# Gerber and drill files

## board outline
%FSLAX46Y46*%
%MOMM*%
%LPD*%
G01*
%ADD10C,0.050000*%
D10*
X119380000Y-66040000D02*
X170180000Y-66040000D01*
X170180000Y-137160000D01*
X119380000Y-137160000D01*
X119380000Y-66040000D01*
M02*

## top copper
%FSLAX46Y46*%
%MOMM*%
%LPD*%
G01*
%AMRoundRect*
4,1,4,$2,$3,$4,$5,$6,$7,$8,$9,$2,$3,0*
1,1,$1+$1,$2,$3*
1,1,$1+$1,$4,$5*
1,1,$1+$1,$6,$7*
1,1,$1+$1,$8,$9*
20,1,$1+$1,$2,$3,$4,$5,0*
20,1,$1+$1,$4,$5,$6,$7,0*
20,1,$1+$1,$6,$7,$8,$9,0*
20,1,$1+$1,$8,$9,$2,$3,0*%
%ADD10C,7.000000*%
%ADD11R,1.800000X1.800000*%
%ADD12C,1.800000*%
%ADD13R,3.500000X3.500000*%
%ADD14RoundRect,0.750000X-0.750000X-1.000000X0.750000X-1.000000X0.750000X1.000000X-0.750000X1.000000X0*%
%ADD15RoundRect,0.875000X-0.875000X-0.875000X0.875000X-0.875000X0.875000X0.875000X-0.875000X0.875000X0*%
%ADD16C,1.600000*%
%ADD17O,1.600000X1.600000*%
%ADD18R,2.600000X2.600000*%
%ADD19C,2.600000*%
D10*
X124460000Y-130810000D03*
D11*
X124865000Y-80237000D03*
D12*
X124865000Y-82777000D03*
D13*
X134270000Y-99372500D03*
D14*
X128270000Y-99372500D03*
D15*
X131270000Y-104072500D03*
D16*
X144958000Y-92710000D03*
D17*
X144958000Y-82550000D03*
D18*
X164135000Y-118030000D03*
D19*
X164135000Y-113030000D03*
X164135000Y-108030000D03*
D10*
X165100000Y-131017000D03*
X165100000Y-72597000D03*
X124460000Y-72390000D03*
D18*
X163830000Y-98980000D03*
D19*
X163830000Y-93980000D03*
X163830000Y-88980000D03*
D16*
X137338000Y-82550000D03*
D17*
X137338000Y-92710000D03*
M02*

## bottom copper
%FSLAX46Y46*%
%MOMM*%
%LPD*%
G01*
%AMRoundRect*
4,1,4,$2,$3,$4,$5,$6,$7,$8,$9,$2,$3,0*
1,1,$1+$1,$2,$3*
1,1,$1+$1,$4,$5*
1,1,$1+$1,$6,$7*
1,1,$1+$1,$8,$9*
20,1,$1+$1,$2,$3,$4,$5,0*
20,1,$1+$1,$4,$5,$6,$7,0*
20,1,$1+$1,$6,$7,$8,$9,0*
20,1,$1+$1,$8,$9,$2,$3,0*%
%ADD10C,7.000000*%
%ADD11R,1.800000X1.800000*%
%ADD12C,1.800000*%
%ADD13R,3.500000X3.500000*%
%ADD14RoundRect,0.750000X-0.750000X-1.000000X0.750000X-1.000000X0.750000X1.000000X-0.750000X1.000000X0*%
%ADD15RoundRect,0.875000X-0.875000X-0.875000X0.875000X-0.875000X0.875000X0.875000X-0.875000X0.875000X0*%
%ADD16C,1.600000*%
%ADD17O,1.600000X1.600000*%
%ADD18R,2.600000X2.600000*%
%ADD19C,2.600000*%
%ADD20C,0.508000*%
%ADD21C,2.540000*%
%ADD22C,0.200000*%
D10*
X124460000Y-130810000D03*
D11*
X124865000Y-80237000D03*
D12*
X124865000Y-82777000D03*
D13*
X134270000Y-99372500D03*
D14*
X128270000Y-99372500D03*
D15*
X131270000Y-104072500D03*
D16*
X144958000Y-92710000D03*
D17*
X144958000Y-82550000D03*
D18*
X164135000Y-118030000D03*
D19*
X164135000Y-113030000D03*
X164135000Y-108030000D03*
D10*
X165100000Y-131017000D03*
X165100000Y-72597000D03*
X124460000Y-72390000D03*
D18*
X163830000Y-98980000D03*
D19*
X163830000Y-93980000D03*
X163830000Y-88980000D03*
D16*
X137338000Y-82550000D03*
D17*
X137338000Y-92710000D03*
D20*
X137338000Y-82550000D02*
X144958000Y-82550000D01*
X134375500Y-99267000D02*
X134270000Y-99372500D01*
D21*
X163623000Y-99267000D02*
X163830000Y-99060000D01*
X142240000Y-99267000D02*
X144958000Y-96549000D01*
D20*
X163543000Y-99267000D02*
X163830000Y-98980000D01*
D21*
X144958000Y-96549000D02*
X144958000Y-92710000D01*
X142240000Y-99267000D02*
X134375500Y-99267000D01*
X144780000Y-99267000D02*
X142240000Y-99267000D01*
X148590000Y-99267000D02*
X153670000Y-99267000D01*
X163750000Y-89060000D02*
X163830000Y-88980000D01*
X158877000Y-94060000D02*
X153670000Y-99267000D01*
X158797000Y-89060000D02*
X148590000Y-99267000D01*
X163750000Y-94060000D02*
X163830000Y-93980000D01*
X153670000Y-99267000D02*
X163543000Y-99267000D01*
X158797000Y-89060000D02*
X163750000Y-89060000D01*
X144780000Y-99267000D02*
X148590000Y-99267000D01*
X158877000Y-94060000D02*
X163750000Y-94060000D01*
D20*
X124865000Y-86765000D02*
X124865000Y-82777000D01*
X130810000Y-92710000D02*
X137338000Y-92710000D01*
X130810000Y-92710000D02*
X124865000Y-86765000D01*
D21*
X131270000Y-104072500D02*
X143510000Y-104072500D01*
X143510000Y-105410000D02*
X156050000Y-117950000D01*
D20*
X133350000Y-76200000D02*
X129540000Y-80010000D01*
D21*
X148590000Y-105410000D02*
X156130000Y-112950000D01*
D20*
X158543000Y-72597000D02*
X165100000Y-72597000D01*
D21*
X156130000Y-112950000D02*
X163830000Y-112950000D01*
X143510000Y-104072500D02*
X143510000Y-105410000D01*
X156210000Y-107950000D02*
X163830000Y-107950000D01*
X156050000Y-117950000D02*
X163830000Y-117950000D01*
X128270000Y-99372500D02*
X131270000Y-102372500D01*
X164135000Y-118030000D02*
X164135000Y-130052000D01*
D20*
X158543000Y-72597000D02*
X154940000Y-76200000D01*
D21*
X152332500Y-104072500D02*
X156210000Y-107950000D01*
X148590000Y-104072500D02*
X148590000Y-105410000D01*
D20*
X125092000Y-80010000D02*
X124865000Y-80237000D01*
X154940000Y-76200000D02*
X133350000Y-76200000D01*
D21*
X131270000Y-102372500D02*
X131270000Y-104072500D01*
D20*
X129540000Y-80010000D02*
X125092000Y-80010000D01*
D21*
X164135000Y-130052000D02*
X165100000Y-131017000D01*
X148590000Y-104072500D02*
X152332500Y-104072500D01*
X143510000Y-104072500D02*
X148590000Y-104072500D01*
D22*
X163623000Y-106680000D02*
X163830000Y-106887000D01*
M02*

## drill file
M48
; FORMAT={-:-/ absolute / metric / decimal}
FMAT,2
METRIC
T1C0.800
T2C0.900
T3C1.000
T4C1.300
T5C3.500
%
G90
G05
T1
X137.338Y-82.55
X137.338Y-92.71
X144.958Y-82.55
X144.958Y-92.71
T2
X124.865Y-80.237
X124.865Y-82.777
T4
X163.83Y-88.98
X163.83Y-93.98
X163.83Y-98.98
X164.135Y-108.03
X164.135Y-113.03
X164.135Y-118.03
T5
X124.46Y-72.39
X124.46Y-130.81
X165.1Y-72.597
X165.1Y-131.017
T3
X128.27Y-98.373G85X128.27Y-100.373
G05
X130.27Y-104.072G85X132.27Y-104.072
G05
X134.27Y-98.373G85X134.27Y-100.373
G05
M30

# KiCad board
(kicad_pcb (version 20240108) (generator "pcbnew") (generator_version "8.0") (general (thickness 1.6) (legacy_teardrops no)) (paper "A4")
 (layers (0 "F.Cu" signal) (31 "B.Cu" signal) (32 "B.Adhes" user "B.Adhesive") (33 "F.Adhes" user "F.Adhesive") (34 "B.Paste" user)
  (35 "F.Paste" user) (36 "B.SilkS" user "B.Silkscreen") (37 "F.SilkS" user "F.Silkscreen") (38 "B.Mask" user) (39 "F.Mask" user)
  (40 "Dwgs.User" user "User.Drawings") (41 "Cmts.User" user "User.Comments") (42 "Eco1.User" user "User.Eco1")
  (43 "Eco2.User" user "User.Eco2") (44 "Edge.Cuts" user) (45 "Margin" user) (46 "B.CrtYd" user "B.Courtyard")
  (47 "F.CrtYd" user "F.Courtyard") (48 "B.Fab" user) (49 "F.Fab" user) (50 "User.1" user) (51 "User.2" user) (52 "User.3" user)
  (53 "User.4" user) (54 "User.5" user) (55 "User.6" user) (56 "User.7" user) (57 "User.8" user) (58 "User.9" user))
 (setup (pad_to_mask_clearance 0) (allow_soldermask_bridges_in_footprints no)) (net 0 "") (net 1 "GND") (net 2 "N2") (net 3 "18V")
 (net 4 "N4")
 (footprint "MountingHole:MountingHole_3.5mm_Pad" (layer "F.Cu") (at 124.46 130.81)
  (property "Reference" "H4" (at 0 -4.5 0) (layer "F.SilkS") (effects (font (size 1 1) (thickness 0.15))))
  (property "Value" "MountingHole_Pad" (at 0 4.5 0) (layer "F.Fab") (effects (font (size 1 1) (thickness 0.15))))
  (pad "1" thru_hole circle (at 0 0) (size 7 7) (drill 3.5) (layers "*.Cu" "*.Mask") (remove_unused_layers no) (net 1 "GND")))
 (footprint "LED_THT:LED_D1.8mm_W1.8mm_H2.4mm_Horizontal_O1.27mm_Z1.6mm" (layer "F.Cu") (at 124.865 80.237 -90)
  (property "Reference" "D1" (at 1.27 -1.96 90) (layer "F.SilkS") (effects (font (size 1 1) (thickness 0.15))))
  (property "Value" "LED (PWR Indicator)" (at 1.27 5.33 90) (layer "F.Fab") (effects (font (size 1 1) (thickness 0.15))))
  (pad "1" thru_hole rect (at 0 0 270) (size 1.8 1.8) (drill 0.9) (layers "*.Cu" "*.Mask") (remove_unused_layers no) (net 1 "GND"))
  (pad "2" thru_hole circle (at 2.54 0 270) (size 1.8 1.8) (drill 0.9) (layers "*.Cu" "*.Mask") (remove_unused_layers no) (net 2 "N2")))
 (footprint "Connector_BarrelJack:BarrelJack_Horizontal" (layer "F.Cu") (at 134.27 99.3725)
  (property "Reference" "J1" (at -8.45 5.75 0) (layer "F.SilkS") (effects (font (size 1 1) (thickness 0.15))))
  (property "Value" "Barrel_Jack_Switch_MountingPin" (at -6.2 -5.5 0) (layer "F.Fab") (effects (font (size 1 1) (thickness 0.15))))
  (pad "1" thru_hole rect (at 0 0) (size 3.5 3.5) (drill oval 1 3) (layers "*.Cu" "*.Mask") (remove_unused_layers no) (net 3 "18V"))
  (pad "2" thru_hole roundrect (at -6 0) (size 3 3.5) (drill oval 1 3) (layers "*.Cu" "*.Mask") (remove_unused_layers no)
   (roundrect_rratio 0.25) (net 1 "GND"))
  (pad "3" thru_hole roundrect (at -3 4.7) (size 3.5 3.5) (drill oval 3 1) (layers "*.Cu" "*.Mask") (remove_unused_layers no)
   (roundrect_rratio 0.25) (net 1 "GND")))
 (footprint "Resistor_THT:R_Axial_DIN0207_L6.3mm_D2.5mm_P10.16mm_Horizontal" (layer "F.Cu") (at 144.958 92.71 90)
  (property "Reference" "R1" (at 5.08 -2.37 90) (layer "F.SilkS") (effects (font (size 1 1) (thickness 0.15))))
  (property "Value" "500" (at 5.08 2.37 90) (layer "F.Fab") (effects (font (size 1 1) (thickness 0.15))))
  (pad "1" thru_hole circle (at 0 0 90) (size 1.6 1.6) (drill 0.8) (layers "*.Cu" "*.Mask") (remove_unused_layers no) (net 3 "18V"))
  (pad "2" thru_hole oval (at 10.16 0 90) (size 1.6 1.6) (drill 0.8) (layers "*.Cu" "*.Mask") (remove_unused_layers no) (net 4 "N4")))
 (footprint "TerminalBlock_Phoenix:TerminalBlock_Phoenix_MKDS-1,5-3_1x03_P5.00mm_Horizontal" (layer "F.Cu") (at 164.135 118.03 90)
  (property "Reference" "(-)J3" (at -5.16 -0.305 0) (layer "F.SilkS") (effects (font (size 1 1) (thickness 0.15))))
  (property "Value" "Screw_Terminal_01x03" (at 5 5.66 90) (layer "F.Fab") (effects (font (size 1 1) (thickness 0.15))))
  (pad "1" thru_hole rect (at 0 0 90) (size 2.6 2.6) (drill 1.3) (layers "*.Cu" "*.Mask") (remove_unused_layers no) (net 1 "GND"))
  (pad "2" thru_hole circle (at 5 0 90) (size 2.6 2.6) (drill 1.3) (layers "*.Cu" "*.Mask") (remove_unused_layers no) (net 1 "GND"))
  (pad "3" thru_hole circle (at 10 0 90) (size 2.6 2.6) (drill 1.3) (layers "*.Cu" "*.Mask") (remove_unused_layers no) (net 1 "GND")))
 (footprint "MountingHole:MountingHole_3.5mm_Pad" (layer "F.Cu") (at 165.1 131.017)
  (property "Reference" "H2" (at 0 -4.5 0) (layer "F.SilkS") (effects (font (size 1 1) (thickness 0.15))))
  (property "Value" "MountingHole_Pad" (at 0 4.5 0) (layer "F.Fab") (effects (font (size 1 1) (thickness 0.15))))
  (pad "1" thru_hole circle (at 0 0) (size 7 7) (drill 3.5) (layers "*.Cu" "*.Mask") (remove_unused_layers no) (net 1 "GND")))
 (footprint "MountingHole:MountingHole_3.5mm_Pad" (layer "F.Cu") (at 165.1 72.597)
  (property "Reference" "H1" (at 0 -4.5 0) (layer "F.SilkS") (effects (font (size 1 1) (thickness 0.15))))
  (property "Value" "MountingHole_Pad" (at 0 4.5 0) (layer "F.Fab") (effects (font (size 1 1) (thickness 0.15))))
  (pad "1" thru_hole circle (at 0 0) (size 7 7) (drill 3.5) (layers "*.Cu" "*.Mask") (remove_unused_layers no) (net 1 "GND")))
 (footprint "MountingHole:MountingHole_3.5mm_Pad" (layer "F.Cu") (at 124.46 72.39)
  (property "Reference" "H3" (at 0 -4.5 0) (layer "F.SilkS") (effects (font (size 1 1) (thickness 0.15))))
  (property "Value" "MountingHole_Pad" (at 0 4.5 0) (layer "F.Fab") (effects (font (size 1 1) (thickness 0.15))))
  (pad "1" thru_hole circle (at 0 0) (size 7 7) (drill 3.5) (layers "*.Cu" "*.Mask") (remove_unused_layers no) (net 1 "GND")))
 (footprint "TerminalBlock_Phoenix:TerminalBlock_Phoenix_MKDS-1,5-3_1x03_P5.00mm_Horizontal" (layer "F.Cu") (at 163.83 98.98 90)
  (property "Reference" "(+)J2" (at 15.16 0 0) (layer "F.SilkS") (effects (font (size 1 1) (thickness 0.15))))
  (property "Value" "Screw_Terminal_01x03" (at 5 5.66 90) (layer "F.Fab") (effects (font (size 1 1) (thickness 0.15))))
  (pad "1" thru_hole rect (at 0 0 90) (size 2.6 2.6) (drill 1.3) (layers "*.Cu" "*.Mask") (remove_unused_layers no) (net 3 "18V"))
  (pad "2" thru_hole circle (at 5 0 90) (size 2.6 2.6) (drill 1.3) (layers "*.Cu" "*.Mask") (remove_unused_layers no) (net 3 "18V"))
  (pad "3" thru_hole circle (at 10 0 90) (size 2.6 2.6) (drill 1.3) (layers "*.Cu" "*.Mask") (remove_unused_layers no) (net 3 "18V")))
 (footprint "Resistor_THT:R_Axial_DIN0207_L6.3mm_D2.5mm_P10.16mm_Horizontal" (layer "F.Cu") (at 137.338 82.55 -90)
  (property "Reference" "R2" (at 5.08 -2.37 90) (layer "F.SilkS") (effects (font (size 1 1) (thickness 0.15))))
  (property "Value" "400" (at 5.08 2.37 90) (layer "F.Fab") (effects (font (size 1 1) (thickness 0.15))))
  (pad "1" thru_hole circle (at 0 0 270) (size 1.6 1.6) (drill 0.8) (layers "*.Cu" "*.Mask") (remove_unused_layers no) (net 4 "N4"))
  (pad "2" thru_hole oval (at 10.16 0 270) (size 1.6 1.6) (drill 0.8) (layers "*.Cu" "*.Mask") (remove_unused_layers no) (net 2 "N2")))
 (gr_rect (start 119.38 66.04) (end 170.18 137.16) (stroke (width 0.05) (type default)) (fill none) (layer "Edge.Cuts"))
 (segment (start 137.338 82.55) (end 144.958 82.55) (width 0.508) (layer "B.Cu") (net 4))
 (segment (start 134.3755 99.267) (end 134.27 99.3725) (width 0.508) (layer "B.Cu") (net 3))
 (segment (start 163.623 99.267) (end 163.83 99.06) (width 2.54) (layer "B.Cu") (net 3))
 (segment (start 142.24 99.267) (end 144.958 96.549) (width 2.54) (layer "B.Cu") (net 3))
 (segment (start 163.543 99.267) (end 163.83 98.98) (width 0.508) (layer "B.Cu") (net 3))
 (segment (start 144.958 96.549) (end 144.958 92.71) (width 2.54) (layer "B.Cu") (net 3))
 (segment (start 142.24 99.267) (end 134.3755 99.267) (width 2.54) (layer "B.Cu") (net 3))
 (segment (start 144.78 99.267) (end 142.24 99.267) (width 2.54) (layer "B.Cu") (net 3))
 (segment (start 148.59 99.267) (end 153.67 99.267) (width 2.54) (layer "B.Cu") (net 3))
 (segment (start 163.75 89.06) (end 163.83 88.98) (width 2.54) (layer "B.Cu") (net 3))
 (segment (start 158.877 94.06) (end 153.67 99.267) (width 2.54) (layer "B.Cu") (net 3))
 (segment (start 158.797 89.06) (end 148.59 99.267) (width 2.54) (layer "B.Cu") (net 3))
 (segment (start 163.75 94.06) (end 163.83 93.98) (width 2.54) (layer "B.Cu") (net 3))
 (segment (start 153.67 99.267) (end 163.543 99.267) (width 2.54) (layer "B.Cu") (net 3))
 (segment (start 158.797 89.06) (end 163.75 89.06) (width 2.54) (layer "B.Cu") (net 3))
 (segment (start 144.78 99.267) (end 148.59 99.267) (width 2.54) (layer "B.Cu") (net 3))
 (segment (start 158.877 94.06) (end 163.75 94.06) (width 2.54) (layer "B.Cu") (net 3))
 (segment (start 124.865 86.765) (end 124.865 82.777) (width 0.508) (layer "B.Cu") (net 2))
 (segment (start 130.81 92.71) (end 137.338 92.71) (width 0.508) (layer "B.Cu") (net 2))
 (segment (start 130.81 92.71) (end 124.865 86.765) (width 0.508) (layer "B.Cu") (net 2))
 (segment (start 131.27 104.0725) (end 143.51 104.0725) (width 2.54) (layer "B.Cu") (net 1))
 (segment (start 143.51 105.41) (end 156.05 117.95) (width 2.54) (layer "B.Cu") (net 1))
 (segment (start 133.35 76.2) (end 129.54 80.01) (width 0.508) (layer "B.Cu") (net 1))
 (segment (start 148.59 105.41) (end 156.13 112.95) (width 2.54) (layer "B.Cu") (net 1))
 (segment (start 158.543 72.597) (end 165.1 72.597) (width 0.508) (layer "B.Cu") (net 1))
 (segment (start 156.13 112.95) (end 163.83 112.95) (width 2.54) (layer "B.Cu") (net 1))
 (segment (start 143.51 104.0725) (end 143.51 105.41) (width 2.54) (layer "B.Cu") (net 1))
 (segment (start 156.21 107.95) (end 163.83 107.95) (width 2.54) (layer "B.Cu") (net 1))
 (segment (start 156.05 117.95) (end 163.83 117.95) (width 2.54) (layer "B.Cu") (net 1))
 (segment (start 128.27 99.3725) (end 131.27 102.3725) (width 2.54) (layer "B.Cu") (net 1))
 (segment (start 164.135 118.03) (end 164.135 130.052) (width 2.54) (layer "B.Cu") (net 1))
 (segment (start 158.543 72.597) (end 154.94 76.2) (width 0.508) (layer "B.Cu") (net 1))
 (segment (start 152.3325 104.0725) (end 156.21 107.95) (width 2.54) (layer "B.Cu") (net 1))
 (segment (start 148.59 104.0725) (end 148.59 105.41) (width 2.54) (layer "B.Cu") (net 1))
 (segment (start 125.092 80.01) (end 124.865 80.237) (width 0.508) (layer "B.Cu") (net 1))
 (segment (start 154.94 76.2) (end 133.35 76.2) (width 0.508) (layer "B.Cu") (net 1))
 (segment (start 131.27 102.3725) (end 131.27 104.0725) (width 2.54) (layer "B.Cu") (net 1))
 (segment (start 129.54 80.01) (end 125.092 80.01) (width 0.508) (layer "B.Cu") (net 1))
 (segment (start 164.135 130.052) (end 165.1 131.017) (width 2.54) (layer "B.Cu") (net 1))
 (segment (start 148.59 104.0725) (end 152.3325 104.0725) (width 2.54) (layer "B.Cu") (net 1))
 (segment (start 143.51 104.0725) (end 148.59 104.0725) (width 2.54) (layer "B.Cu") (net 1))
 (segment (start 163.623 106.68) (end 163.83 106.887) (width 0.2) (layer "B.Cu") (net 1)))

